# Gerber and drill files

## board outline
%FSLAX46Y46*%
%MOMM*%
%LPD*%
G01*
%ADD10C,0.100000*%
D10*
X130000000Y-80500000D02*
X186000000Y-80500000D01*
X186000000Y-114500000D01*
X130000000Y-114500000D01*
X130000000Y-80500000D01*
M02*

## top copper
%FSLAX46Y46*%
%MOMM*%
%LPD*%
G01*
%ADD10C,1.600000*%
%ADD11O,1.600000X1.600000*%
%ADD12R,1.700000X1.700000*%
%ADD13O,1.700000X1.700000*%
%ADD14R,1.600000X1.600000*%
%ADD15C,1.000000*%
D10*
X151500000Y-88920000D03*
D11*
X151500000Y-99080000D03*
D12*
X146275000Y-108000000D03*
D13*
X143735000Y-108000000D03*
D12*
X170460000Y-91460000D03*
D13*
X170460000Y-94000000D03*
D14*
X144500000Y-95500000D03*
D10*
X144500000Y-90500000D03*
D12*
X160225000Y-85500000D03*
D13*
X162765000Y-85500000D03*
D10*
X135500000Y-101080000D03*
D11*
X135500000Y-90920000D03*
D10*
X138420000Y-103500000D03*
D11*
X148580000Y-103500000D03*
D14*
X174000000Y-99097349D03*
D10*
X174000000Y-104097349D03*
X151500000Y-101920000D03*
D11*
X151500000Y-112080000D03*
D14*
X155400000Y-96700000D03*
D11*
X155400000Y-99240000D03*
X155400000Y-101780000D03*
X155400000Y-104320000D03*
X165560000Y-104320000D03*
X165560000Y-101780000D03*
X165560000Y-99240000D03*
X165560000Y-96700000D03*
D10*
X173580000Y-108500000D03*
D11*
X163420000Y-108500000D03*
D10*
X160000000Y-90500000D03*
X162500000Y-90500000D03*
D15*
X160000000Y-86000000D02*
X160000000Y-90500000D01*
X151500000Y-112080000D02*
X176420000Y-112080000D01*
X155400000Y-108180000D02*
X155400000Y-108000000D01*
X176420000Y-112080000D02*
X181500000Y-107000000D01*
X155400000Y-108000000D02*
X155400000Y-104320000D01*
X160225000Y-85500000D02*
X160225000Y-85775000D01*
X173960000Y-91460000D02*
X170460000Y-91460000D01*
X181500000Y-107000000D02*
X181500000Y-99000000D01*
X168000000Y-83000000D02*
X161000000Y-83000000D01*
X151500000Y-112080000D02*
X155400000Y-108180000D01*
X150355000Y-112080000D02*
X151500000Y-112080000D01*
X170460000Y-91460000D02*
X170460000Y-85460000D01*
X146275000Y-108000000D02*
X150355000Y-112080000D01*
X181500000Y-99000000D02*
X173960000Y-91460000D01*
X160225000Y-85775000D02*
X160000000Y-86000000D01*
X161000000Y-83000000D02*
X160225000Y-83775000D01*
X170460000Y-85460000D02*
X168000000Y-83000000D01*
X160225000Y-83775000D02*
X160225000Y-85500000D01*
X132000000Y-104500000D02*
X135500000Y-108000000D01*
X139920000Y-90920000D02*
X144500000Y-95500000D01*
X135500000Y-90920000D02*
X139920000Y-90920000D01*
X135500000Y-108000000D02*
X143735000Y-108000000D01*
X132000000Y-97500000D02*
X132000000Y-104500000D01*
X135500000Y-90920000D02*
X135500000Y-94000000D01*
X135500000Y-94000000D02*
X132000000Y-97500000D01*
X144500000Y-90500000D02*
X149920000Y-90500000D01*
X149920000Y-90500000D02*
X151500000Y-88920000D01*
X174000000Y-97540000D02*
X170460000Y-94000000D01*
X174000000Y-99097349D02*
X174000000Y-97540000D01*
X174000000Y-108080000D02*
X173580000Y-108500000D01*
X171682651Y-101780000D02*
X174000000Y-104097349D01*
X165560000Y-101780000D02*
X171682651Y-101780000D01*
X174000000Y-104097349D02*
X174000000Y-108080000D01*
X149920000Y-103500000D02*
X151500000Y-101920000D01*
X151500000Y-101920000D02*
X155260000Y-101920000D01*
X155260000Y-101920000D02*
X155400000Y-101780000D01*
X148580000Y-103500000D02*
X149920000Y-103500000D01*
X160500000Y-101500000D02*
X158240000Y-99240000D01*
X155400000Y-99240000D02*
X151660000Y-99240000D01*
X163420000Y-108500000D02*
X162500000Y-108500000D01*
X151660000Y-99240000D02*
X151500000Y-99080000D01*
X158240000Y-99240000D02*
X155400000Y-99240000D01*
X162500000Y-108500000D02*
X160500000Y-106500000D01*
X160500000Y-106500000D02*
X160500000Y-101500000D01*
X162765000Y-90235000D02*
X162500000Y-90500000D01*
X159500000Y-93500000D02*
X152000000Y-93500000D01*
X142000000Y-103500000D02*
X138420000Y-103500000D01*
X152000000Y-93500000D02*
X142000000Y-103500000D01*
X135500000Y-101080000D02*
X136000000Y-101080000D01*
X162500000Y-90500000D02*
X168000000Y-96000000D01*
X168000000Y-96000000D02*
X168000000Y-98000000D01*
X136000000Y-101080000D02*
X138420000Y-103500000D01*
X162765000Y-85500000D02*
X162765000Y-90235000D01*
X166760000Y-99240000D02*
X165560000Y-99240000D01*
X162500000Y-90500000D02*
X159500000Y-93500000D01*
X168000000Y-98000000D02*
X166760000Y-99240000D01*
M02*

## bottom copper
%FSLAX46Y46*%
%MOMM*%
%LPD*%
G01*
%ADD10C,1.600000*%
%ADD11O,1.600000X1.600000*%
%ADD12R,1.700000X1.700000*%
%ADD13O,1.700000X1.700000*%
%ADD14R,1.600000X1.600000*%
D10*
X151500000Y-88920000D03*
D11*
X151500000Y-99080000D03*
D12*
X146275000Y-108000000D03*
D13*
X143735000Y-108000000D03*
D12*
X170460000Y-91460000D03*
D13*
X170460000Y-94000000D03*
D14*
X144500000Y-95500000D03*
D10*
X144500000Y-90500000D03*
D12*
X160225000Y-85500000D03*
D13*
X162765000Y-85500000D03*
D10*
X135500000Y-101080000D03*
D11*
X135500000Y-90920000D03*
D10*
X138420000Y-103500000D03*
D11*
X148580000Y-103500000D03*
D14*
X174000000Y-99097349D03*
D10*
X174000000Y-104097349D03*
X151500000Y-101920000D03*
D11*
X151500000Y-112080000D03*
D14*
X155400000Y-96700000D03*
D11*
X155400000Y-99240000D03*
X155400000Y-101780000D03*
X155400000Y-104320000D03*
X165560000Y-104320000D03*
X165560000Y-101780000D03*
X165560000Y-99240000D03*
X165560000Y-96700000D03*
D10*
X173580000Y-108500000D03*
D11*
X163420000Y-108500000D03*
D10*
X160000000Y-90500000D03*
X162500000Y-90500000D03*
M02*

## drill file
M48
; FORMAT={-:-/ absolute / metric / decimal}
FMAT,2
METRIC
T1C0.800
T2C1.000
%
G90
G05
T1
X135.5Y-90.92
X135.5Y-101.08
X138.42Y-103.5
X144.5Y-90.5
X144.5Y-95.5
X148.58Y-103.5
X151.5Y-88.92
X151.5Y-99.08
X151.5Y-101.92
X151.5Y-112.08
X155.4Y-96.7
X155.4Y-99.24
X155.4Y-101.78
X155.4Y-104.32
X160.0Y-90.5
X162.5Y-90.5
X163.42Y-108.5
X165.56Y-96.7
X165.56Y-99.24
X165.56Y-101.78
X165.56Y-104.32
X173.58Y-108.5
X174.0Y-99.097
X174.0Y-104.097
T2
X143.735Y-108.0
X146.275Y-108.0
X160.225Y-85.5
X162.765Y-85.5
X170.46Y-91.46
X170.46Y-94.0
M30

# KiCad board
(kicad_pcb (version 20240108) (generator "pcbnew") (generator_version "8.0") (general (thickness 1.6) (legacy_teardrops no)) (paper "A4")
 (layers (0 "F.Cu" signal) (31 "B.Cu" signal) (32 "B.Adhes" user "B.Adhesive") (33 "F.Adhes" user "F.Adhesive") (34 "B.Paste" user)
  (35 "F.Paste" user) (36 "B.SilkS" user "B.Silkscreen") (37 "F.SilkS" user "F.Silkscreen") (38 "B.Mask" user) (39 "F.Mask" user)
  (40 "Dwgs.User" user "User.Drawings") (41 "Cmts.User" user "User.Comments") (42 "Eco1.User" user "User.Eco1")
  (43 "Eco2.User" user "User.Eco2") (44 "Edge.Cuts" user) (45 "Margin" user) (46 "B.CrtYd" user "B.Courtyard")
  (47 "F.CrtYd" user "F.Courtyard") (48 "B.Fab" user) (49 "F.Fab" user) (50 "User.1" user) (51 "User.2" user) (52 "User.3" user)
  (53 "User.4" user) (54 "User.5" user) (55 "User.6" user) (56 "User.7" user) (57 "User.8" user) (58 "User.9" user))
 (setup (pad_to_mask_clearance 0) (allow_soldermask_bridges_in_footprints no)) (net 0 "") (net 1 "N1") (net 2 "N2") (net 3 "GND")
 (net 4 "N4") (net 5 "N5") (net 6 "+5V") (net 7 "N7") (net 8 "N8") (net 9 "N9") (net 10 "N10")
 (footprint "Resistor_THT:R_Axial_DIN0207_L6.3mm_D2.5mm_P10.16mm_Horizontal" (layer "F.Cu") (at 151.5 88.92 -90)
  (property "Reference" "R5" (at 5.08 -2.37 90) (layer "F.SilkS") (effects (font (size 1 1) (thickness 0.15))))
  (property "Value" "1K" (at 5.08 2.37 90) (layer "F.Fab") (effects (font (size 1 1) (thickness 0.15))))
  (pad "1" thru_hole circle (at 0 0 270) (size 1.6 1.6) (drill 0.8) (layers "*.Cu" "*.Mask") (remove_unused_layers no) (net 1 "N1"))
  (pad "2" thru_hole oval (at 10.16 0 270) (size 1.6 1.6) (drill 0.8) (layers "*.Cu" "*.Mask") (remove_unused_layers no) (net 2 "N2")))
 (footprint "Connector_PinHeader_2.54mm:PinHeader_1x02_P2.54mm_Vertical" (layer "F.Cu") (at 146.275 108 -90)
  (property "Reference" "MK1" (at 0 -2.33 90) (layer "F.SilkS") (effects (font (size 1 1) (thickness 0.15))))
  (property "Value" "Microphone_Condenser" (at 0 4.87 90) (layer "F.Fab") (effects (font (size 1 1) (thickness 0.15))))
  (pad "1" thru_hole rect (at 0 0 270) (size 1.7 1.7) (drill 1) (layers "*.Cu" "*.Mask") (remove_unused_layers no) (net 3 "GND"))
  (pad "2" thru_hole oval (at 0 2.54 270) (size 1.7 1.7) (drill 1) (layers "*.Cu" "*.Mask") (remove_unused_layers no) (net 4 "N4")))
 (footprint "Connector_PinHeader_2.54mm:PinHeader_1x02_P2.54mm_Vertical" (layer "F.Cu") (at 170.46 91.46)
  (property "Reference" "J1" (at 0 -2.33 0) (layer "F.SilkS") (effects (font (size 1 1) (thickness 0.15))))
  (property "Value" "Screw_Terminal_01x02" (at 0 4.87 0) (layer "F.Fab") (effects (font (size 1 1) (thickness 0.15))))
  (pad "1" thru_hole rect (at 0 0) (size 1.7 1.7) (drill 1) (layers "*.Cu" "*.Mask") (remove_unused_layers no) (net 3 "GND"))
  (pad "2" thru_hole oval (at 0 2.54) (size 1.7 1.7) (drill 1) (layers "*.Cu" "*.Mask") (remove_unused_layers no) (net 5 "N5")))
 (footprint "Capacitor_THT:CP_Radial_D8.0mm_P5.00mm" (layer "F.Cu") (at 144.5 95.5 90)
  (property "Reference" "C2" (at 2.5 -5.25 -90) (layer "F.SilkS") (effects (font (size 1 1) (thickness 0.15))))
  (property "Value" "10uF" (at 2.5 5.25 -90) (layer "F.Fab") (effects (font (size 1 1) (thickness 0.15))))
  (pad "1" thru_hole rect (at 0 0 90) (size 1.6 1.6) (drill 0.8) (layers "*.Cu" "*.Mask") (remove_unused_layers no) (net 4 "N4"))
  (pad "2" thru_hole circle (at 5 0 90) (size 1.6 1.6) (drill 0.8) (layers "*.Cu" "*.Mask") (remove_unused_layers no) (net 1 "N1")))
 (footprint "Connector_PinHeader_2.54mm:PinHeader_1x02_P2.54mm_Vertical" (layer "F.Cu") (at 160.225 85.5 90)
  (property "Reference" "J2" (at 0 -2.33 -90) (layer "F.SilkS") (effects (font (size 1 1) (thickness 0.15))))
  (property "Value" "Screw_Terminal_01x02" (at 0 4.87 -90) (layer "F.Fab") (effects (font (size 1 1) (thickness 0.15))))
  (pad "1" thru_hole rect (at 0 0 90) (size 1.7 1.7) (drill 1) (layers "*.Cu" "*.Mask") (remove_unused_layers no) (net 3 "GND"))
  (pad "2" thru_hole oval (at 0 2.54 90) (size 1.7 1.7) (drill 1) (layers "*.Cu" "*.Mask") (remove_unused_layers no) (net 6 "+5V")))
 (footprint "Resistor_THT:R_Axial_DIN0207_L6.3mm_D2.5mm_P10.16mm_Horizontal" (layer "F.Cu") (at 135.5 101.08 90)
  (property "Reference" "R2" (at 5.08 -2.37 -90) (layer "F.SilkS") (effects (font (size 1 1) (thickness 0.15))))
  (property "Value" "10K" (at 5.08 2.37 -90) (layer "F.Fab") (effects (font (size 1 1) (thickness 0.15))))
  (pad "1" thru_hole circle (at 0 0 90) (size 1.6 1.6) (drill 0.8) (layers "*.Cu" "*.Mask") (remove_unused_layers no) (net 6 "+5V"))
  (pad "2" thru_hole oval (at 10.16 0 90) (size 1.6 1.6) (drill 0.8) (layers "*.Cu" "*.Mask") (remove_unused_layers no) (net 4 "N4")))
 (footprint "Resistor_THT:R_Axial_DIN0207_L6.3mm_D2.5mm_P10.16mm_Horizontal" (layer "F.Cu") (at 138.42 103.5)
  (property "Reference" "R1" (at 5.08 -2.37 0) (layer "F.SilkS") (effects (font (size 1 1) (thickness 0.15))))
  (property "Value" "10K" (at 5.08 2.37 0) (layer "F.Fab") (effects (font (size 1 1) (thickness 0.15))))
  (pad "1" thru_hole circle (at 0 0) (size 1.6 1.6) (drill 0.8) (layers "*.Cu" "*.Mask") (remove_unused_layers no) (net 6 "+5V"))
  (pad "2" thru_hole oval (at 10.16 0) (size 1.6 1.6) (drill 0.8) (layers "*.Cu" "*.Mask") (remove_unused_layers no) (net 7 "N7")))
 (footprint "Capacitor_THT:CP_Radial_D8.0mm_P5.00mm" (layer "F.Cu") (at 174 99.097349 -90)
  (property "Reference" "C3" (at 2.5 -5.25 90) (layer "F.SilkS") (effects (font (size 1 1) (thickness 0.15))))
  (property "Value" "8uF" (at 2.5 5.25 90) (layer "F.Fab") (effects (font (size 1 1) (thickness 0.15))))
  (pad "1" thru_hole rect (at 0 0 270) (size 1.6 1.6) (drill 0.8) (layers "*.Cu" "*.Mask") (remove_unused_layers no) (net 5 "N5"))
  (pad "2" thru_hole circle (at 5 0 270) (size 1.6 1.6) (drill 0.8) (layers "*.Cu" "*.Mask") (remove_unused_layers no) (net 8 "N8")))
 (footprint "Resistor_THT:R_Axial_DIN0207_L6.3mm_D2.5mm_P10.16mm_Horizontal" (layer "F.Cu") (at 151.5 101.92 -90)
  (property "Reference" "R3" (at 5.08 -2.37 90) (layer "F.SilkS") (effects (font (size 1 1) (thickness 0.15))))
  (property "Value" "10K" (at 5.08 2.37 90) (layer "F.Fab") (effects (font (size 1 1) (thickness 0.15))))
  (pad "1" thru_hole circle (at 0 0 270) (size 1.6 1.6) (drill 0.8) (layers "*.Cu" "*.Mask") (remove_unused_layers no) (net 7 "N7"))
  (pad "2" thru_hole oval (at 10.16 0 270) (size 1.6 1.6) (drill 0.8) (layers "*.Cu" "*.Mask") (remove_unused_layers no) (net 3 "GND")))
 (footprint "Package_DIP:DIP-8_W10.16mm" (layer "F.Cu") (at 155.4 96.7)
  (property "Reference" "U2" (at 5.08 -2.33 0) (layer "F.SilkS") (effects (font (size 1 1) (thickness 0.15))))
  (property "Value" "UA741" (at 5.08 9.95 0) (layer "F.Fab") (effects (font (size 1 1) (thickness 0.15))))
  (pad "1" thru_hole rect (at 0 0) (size 1.6 1.6) (drill 0.8) (layers "*.Cu" "*.Mask") (remove_unused_layers no) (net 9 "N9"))
  (pad "2" thru_hole oval (at 0 2.54) (size 1.6 1.6) (drill 0.8) (layers "*.Cu" "*.Mask") (remove_unused_layers no) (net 2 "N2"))
  (pad "3" thru_hole oval (at 0 5.08) (size 1.6 1.6) (drill 0.8) (layers "*.Cu" "*.Mask") (remove_unused_layers no) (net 7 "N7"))
  (pad "4" thru_hole oval (at 0 7.62) (size 1.6 1.6) (drill 0.8) (layers "*.Cu" "*.Mask") (remove_unused_layers no) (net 3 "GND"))
  (pad "5" thru_hole oval (at 10.16 7.62) (size 1.6 1.6) (drill 0.8) (layers "*.Cu" "*.Mask") (remove_unused_layers no) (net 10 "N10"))
  (pad "6" thru_hole oval (at 10.16 5.08) (size 1.6 1.6) (drill 0.8) (layers "*.Cu" "*.Mask") (remove_unused_layers no) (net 8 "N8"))
  (pad "7" thru_hole oval (at 10.16 2.54) (size 1.6 1.6) (drill 0.8) (layers "*.Cu" "*.Mask") (remove_unused_layers no) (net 6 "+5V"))
  (pad "8" thru_hole oval (at 10.16 0) (size 1.6 1.6) (drill 0.8) (layers "*.Cu" "*.Mask") (remove_unused_layers no)))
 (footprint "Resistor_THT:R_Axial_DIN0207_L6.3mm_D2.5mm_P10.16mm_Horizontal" (layer "F.Cu") (at 173.58 108.5 180)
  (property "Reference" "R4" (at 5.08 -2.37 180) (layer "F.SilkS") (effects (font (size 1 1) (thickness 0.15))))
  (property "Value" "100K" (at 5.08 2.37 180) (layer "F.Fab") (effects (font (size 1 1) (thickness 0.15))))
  (pad "1" thru_hole circle (at 0 0 180) (size 1.6 1.6) (drill 0.8) (layers "*.Cu" "*.Mask") (remove_unused_layers no) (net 8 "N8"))
  (pad "2" thru_hole oval (at 10.16 0 180) (size 1.6 1.6) (drill 0.8) (layers "*.Cu" "*.Mask") (remove_unused_layers no) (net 2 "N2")))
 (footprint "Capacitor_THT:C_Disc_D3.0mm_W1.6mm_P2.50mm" (layer "F.Cu") (at 160 90.5)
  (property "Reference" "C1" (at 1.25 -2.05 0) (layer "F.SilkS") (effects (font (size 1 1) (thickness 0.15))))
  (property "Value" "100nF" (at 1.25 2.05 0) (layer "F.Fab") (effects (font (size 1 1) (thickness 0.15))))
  (pad "1" thru_hole circle (at 0 0) (size 1.6 1.6) (drill 0.8) (layers "*.Cu" "*.Mask") (remove_unused_layers no) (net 3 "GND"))
  (pad "2" thru_hole circle (at 2.5 0) (size 1.6 1.6) (drill 0.8) (layers "*.Cu" "*.Mask") (remove_unused_layers no) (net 6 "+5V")))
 (gr_rect (start 130 80.5) (end 186 114.5) (stroke (width 0.1) (type default)) (fill none) (layer "Edge.Cuts"))
 (segment (start 160 86) (end 160 90.5) (width 1) (layer "F.Cu") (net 3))
 (segment (start 151.5 112.08) (end 176.42 112.08) (width 1) (layer "F.Cu") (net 3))
 (segment (start 155.4 108.18) (end 155.4 108) (width 1) (layer "F.Cu") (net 3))
 (segment (start 176.42 112.08) (end 181.5 107) (width 1) (layer "F.Cu") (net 3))
 (segment (start 155.4 108) (end 155.4 104.32) (width 1) (layer "F.Cu") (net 3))
 (segment (start 160.225 85.5) (end 160.225 85.775) (width 1) (layer "F.Cu") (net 3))
 (segment (start 173.96 91.46) (end 170.46 91.46) (width 1) (layer "F.Cu") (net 3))
 (segment (start 181.5 107) (end 181.5 99) (width 1) (layer "F.Cu") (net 3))
 (segment (start 168 83) (end 161 83) (width 1) (layer "F.Cu") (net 3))
 (segment (start 151.5 112.08) (end 155.4 108.18) (width 1) (layer "F.Cu") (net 3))
 (segment (start 150.355 112.08) (end 151.5 112.08) (width 1) (layer "F.Cu") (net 3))
 (segment (start 170.46 91.46) (end 170.46 85.46) (width 1) (layer "F.Cu") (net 3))
 (segment (start 146.275 108) (end 150.355 112.08) (width 1) (layer "F.Cu") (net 3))
 (segment (start 181.5 99) (end 173.96 91.46) (width 1) (layer "F.Cu") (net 3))
 (segment (start 160.225 85.775) (end 160 86) (width 1) (layer "F.Cu") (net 3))
 (segment (start 161 83) (end 160.225 83.775) (width 1) (layer "F.Cu") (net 3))
 (segment (start 170.46 85.46) (end 168 83) (width 1) (layer "F.Cu") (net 3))
 (segment (start 160.225 83.775) (end 160.225 85.5) (width 1) (layer "F.Cu") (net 3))
 (segment (start 132 104.5) (end 135.5 108) (width 1) (layer "F.Cu") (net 4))
 (segment (start 139.92 90.92) (end 144.5 95.5) (width 1) (layer "F.Cu") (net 4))
 (segment (start 135.5 90.92) (end 139.92 90.92) (width 1) (layer "F.Cu") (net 4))
 (segment (start 135.5 108) (end 143.735 108) (width 1) (layer "F.Cu") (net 4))
 (segment (start 132 97.5) (end 132 104.5) (width 1) (layer "F.Cu") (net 4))
 (segment (start 135.5 90.92) (end 135.5 94) (width 1) (layer "F.Cu") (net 4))
 (segment (start 135.5 94) (end 132 97.5) (width 1) (layer "F.Cu") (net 4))
 (segment (start 144.5 90.5) (end 149.92 90.5) (width 1) (layer "F.Cu") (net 1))
 (segment (start 149.92 90.5) (end 151.5 88.92) (width 1) (layer "F.Cu") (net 1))
 (segment (start 174 97.54) (end 170.46 94) (width 1) (layer "F.Cu") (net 5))
 (segment (start 174 99.097349) (end 174 97.54) (width 1) (layer "F.Cu") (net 5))
 (segment (start 174 108.08) (end 173.58 108.5) (width 1) (layer "F.Cu") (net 8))
 (segment (start 171.682651 101.78) (end 174 104.097349) (width 1) (layer "F.Cu") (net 8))
 (segment (start 165.56 101.78) (end 171.682651 101.78) (width 1) (layer "F.Cu") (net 8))
 (segment (start 174 104.097349) (end 174 108.08) (width 1) (layer "F.Cu") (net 8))
 (segment (start 149.92 103.5) (end 151.5 101.92) (width 1) (layer "F.Cu") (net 7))
 (segment (start 151.5 101.92) (end 155.26 101.92) (width 1) (layer "F.Cu") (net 7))
 (segment (start 155.26 101.92) (end 155.4 101.78) (width 1) (layer "F.Cu") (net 7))
 (segment (start 148.58 103.5) (end 149.92 103.5) (width 1) (layer "F.Cu") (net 7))
 (segment (start 160.5 101.5) (end 158.24 99.24) (width 1) (layer "F.Cu") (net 2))
 (segment (start 155.4 99.24) (end 151.66 99.24) (width 1) (layer "F.Cu") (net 2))
 (segment (start 163.42 108.5) (end 162.5 108.5) (width 1) (layer "F.Cu") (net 2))
 (segment (start 151.66 99.24) (end 151.5 99.08) (width 1) (layer "F.Cu") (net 2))
 (segment (start 158.24 99.24) (end 155.4 99.24) (width 1) (layer "F.Cu") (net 2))
 (segment (start 162.5 108.5) (end 160.5 106.5) (width 1) (layer "F.Cu") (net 2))
 (segment (start 160.5 106.5) (end 160.5 101.5) (width 1) (layer "F.Cu") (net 2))
 (segment (start 162.765 90.235) (end 162.5 90.5) (width 1) (layer "F.Cu") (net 6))
 (segment (start 159.5 93.5) (end 152 93.5) (width 1) (layer "F.Cu") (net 6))
 (segment (start 142 103.5) (end 138.42 103.5) (width 1) (layer "F.Cu") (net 6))
 (segment (start 152 93.5) (end 142 103.5) (width 1) (layer "F.Cu") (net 6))
 (segment (start 135.5 101.08) (end 136 101.08) (width 1) (layer "F.Cu") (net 6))
 (segment (start 162.5 90.5) (end 168 96) (width 1) (layer "F.Cu") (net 6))
 (segment (start 168 96) (end 168 98) (width 1) (layer "F.Cu") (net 6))
 (segment (start 136 101.08) (end 138.42 103.5) (width 1) (layer "F.Cu") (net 6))
 (segment (start 162.765 85.5) (end 162.765 90.235) (width 1) (layer "F.Cu") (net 6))
 (segment (start 166.76 99.24) (end 165.56 99.24) (width 1) (layer "F.Cu") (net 6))
 (segment (start 162.5 90.5) (end 159.5 93.5) (width 1) (layer "F.Cu") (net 6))
 (segment (start 168 98) (end 166.76 99.24) (width 1) (layer "F.Cu") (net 6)))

